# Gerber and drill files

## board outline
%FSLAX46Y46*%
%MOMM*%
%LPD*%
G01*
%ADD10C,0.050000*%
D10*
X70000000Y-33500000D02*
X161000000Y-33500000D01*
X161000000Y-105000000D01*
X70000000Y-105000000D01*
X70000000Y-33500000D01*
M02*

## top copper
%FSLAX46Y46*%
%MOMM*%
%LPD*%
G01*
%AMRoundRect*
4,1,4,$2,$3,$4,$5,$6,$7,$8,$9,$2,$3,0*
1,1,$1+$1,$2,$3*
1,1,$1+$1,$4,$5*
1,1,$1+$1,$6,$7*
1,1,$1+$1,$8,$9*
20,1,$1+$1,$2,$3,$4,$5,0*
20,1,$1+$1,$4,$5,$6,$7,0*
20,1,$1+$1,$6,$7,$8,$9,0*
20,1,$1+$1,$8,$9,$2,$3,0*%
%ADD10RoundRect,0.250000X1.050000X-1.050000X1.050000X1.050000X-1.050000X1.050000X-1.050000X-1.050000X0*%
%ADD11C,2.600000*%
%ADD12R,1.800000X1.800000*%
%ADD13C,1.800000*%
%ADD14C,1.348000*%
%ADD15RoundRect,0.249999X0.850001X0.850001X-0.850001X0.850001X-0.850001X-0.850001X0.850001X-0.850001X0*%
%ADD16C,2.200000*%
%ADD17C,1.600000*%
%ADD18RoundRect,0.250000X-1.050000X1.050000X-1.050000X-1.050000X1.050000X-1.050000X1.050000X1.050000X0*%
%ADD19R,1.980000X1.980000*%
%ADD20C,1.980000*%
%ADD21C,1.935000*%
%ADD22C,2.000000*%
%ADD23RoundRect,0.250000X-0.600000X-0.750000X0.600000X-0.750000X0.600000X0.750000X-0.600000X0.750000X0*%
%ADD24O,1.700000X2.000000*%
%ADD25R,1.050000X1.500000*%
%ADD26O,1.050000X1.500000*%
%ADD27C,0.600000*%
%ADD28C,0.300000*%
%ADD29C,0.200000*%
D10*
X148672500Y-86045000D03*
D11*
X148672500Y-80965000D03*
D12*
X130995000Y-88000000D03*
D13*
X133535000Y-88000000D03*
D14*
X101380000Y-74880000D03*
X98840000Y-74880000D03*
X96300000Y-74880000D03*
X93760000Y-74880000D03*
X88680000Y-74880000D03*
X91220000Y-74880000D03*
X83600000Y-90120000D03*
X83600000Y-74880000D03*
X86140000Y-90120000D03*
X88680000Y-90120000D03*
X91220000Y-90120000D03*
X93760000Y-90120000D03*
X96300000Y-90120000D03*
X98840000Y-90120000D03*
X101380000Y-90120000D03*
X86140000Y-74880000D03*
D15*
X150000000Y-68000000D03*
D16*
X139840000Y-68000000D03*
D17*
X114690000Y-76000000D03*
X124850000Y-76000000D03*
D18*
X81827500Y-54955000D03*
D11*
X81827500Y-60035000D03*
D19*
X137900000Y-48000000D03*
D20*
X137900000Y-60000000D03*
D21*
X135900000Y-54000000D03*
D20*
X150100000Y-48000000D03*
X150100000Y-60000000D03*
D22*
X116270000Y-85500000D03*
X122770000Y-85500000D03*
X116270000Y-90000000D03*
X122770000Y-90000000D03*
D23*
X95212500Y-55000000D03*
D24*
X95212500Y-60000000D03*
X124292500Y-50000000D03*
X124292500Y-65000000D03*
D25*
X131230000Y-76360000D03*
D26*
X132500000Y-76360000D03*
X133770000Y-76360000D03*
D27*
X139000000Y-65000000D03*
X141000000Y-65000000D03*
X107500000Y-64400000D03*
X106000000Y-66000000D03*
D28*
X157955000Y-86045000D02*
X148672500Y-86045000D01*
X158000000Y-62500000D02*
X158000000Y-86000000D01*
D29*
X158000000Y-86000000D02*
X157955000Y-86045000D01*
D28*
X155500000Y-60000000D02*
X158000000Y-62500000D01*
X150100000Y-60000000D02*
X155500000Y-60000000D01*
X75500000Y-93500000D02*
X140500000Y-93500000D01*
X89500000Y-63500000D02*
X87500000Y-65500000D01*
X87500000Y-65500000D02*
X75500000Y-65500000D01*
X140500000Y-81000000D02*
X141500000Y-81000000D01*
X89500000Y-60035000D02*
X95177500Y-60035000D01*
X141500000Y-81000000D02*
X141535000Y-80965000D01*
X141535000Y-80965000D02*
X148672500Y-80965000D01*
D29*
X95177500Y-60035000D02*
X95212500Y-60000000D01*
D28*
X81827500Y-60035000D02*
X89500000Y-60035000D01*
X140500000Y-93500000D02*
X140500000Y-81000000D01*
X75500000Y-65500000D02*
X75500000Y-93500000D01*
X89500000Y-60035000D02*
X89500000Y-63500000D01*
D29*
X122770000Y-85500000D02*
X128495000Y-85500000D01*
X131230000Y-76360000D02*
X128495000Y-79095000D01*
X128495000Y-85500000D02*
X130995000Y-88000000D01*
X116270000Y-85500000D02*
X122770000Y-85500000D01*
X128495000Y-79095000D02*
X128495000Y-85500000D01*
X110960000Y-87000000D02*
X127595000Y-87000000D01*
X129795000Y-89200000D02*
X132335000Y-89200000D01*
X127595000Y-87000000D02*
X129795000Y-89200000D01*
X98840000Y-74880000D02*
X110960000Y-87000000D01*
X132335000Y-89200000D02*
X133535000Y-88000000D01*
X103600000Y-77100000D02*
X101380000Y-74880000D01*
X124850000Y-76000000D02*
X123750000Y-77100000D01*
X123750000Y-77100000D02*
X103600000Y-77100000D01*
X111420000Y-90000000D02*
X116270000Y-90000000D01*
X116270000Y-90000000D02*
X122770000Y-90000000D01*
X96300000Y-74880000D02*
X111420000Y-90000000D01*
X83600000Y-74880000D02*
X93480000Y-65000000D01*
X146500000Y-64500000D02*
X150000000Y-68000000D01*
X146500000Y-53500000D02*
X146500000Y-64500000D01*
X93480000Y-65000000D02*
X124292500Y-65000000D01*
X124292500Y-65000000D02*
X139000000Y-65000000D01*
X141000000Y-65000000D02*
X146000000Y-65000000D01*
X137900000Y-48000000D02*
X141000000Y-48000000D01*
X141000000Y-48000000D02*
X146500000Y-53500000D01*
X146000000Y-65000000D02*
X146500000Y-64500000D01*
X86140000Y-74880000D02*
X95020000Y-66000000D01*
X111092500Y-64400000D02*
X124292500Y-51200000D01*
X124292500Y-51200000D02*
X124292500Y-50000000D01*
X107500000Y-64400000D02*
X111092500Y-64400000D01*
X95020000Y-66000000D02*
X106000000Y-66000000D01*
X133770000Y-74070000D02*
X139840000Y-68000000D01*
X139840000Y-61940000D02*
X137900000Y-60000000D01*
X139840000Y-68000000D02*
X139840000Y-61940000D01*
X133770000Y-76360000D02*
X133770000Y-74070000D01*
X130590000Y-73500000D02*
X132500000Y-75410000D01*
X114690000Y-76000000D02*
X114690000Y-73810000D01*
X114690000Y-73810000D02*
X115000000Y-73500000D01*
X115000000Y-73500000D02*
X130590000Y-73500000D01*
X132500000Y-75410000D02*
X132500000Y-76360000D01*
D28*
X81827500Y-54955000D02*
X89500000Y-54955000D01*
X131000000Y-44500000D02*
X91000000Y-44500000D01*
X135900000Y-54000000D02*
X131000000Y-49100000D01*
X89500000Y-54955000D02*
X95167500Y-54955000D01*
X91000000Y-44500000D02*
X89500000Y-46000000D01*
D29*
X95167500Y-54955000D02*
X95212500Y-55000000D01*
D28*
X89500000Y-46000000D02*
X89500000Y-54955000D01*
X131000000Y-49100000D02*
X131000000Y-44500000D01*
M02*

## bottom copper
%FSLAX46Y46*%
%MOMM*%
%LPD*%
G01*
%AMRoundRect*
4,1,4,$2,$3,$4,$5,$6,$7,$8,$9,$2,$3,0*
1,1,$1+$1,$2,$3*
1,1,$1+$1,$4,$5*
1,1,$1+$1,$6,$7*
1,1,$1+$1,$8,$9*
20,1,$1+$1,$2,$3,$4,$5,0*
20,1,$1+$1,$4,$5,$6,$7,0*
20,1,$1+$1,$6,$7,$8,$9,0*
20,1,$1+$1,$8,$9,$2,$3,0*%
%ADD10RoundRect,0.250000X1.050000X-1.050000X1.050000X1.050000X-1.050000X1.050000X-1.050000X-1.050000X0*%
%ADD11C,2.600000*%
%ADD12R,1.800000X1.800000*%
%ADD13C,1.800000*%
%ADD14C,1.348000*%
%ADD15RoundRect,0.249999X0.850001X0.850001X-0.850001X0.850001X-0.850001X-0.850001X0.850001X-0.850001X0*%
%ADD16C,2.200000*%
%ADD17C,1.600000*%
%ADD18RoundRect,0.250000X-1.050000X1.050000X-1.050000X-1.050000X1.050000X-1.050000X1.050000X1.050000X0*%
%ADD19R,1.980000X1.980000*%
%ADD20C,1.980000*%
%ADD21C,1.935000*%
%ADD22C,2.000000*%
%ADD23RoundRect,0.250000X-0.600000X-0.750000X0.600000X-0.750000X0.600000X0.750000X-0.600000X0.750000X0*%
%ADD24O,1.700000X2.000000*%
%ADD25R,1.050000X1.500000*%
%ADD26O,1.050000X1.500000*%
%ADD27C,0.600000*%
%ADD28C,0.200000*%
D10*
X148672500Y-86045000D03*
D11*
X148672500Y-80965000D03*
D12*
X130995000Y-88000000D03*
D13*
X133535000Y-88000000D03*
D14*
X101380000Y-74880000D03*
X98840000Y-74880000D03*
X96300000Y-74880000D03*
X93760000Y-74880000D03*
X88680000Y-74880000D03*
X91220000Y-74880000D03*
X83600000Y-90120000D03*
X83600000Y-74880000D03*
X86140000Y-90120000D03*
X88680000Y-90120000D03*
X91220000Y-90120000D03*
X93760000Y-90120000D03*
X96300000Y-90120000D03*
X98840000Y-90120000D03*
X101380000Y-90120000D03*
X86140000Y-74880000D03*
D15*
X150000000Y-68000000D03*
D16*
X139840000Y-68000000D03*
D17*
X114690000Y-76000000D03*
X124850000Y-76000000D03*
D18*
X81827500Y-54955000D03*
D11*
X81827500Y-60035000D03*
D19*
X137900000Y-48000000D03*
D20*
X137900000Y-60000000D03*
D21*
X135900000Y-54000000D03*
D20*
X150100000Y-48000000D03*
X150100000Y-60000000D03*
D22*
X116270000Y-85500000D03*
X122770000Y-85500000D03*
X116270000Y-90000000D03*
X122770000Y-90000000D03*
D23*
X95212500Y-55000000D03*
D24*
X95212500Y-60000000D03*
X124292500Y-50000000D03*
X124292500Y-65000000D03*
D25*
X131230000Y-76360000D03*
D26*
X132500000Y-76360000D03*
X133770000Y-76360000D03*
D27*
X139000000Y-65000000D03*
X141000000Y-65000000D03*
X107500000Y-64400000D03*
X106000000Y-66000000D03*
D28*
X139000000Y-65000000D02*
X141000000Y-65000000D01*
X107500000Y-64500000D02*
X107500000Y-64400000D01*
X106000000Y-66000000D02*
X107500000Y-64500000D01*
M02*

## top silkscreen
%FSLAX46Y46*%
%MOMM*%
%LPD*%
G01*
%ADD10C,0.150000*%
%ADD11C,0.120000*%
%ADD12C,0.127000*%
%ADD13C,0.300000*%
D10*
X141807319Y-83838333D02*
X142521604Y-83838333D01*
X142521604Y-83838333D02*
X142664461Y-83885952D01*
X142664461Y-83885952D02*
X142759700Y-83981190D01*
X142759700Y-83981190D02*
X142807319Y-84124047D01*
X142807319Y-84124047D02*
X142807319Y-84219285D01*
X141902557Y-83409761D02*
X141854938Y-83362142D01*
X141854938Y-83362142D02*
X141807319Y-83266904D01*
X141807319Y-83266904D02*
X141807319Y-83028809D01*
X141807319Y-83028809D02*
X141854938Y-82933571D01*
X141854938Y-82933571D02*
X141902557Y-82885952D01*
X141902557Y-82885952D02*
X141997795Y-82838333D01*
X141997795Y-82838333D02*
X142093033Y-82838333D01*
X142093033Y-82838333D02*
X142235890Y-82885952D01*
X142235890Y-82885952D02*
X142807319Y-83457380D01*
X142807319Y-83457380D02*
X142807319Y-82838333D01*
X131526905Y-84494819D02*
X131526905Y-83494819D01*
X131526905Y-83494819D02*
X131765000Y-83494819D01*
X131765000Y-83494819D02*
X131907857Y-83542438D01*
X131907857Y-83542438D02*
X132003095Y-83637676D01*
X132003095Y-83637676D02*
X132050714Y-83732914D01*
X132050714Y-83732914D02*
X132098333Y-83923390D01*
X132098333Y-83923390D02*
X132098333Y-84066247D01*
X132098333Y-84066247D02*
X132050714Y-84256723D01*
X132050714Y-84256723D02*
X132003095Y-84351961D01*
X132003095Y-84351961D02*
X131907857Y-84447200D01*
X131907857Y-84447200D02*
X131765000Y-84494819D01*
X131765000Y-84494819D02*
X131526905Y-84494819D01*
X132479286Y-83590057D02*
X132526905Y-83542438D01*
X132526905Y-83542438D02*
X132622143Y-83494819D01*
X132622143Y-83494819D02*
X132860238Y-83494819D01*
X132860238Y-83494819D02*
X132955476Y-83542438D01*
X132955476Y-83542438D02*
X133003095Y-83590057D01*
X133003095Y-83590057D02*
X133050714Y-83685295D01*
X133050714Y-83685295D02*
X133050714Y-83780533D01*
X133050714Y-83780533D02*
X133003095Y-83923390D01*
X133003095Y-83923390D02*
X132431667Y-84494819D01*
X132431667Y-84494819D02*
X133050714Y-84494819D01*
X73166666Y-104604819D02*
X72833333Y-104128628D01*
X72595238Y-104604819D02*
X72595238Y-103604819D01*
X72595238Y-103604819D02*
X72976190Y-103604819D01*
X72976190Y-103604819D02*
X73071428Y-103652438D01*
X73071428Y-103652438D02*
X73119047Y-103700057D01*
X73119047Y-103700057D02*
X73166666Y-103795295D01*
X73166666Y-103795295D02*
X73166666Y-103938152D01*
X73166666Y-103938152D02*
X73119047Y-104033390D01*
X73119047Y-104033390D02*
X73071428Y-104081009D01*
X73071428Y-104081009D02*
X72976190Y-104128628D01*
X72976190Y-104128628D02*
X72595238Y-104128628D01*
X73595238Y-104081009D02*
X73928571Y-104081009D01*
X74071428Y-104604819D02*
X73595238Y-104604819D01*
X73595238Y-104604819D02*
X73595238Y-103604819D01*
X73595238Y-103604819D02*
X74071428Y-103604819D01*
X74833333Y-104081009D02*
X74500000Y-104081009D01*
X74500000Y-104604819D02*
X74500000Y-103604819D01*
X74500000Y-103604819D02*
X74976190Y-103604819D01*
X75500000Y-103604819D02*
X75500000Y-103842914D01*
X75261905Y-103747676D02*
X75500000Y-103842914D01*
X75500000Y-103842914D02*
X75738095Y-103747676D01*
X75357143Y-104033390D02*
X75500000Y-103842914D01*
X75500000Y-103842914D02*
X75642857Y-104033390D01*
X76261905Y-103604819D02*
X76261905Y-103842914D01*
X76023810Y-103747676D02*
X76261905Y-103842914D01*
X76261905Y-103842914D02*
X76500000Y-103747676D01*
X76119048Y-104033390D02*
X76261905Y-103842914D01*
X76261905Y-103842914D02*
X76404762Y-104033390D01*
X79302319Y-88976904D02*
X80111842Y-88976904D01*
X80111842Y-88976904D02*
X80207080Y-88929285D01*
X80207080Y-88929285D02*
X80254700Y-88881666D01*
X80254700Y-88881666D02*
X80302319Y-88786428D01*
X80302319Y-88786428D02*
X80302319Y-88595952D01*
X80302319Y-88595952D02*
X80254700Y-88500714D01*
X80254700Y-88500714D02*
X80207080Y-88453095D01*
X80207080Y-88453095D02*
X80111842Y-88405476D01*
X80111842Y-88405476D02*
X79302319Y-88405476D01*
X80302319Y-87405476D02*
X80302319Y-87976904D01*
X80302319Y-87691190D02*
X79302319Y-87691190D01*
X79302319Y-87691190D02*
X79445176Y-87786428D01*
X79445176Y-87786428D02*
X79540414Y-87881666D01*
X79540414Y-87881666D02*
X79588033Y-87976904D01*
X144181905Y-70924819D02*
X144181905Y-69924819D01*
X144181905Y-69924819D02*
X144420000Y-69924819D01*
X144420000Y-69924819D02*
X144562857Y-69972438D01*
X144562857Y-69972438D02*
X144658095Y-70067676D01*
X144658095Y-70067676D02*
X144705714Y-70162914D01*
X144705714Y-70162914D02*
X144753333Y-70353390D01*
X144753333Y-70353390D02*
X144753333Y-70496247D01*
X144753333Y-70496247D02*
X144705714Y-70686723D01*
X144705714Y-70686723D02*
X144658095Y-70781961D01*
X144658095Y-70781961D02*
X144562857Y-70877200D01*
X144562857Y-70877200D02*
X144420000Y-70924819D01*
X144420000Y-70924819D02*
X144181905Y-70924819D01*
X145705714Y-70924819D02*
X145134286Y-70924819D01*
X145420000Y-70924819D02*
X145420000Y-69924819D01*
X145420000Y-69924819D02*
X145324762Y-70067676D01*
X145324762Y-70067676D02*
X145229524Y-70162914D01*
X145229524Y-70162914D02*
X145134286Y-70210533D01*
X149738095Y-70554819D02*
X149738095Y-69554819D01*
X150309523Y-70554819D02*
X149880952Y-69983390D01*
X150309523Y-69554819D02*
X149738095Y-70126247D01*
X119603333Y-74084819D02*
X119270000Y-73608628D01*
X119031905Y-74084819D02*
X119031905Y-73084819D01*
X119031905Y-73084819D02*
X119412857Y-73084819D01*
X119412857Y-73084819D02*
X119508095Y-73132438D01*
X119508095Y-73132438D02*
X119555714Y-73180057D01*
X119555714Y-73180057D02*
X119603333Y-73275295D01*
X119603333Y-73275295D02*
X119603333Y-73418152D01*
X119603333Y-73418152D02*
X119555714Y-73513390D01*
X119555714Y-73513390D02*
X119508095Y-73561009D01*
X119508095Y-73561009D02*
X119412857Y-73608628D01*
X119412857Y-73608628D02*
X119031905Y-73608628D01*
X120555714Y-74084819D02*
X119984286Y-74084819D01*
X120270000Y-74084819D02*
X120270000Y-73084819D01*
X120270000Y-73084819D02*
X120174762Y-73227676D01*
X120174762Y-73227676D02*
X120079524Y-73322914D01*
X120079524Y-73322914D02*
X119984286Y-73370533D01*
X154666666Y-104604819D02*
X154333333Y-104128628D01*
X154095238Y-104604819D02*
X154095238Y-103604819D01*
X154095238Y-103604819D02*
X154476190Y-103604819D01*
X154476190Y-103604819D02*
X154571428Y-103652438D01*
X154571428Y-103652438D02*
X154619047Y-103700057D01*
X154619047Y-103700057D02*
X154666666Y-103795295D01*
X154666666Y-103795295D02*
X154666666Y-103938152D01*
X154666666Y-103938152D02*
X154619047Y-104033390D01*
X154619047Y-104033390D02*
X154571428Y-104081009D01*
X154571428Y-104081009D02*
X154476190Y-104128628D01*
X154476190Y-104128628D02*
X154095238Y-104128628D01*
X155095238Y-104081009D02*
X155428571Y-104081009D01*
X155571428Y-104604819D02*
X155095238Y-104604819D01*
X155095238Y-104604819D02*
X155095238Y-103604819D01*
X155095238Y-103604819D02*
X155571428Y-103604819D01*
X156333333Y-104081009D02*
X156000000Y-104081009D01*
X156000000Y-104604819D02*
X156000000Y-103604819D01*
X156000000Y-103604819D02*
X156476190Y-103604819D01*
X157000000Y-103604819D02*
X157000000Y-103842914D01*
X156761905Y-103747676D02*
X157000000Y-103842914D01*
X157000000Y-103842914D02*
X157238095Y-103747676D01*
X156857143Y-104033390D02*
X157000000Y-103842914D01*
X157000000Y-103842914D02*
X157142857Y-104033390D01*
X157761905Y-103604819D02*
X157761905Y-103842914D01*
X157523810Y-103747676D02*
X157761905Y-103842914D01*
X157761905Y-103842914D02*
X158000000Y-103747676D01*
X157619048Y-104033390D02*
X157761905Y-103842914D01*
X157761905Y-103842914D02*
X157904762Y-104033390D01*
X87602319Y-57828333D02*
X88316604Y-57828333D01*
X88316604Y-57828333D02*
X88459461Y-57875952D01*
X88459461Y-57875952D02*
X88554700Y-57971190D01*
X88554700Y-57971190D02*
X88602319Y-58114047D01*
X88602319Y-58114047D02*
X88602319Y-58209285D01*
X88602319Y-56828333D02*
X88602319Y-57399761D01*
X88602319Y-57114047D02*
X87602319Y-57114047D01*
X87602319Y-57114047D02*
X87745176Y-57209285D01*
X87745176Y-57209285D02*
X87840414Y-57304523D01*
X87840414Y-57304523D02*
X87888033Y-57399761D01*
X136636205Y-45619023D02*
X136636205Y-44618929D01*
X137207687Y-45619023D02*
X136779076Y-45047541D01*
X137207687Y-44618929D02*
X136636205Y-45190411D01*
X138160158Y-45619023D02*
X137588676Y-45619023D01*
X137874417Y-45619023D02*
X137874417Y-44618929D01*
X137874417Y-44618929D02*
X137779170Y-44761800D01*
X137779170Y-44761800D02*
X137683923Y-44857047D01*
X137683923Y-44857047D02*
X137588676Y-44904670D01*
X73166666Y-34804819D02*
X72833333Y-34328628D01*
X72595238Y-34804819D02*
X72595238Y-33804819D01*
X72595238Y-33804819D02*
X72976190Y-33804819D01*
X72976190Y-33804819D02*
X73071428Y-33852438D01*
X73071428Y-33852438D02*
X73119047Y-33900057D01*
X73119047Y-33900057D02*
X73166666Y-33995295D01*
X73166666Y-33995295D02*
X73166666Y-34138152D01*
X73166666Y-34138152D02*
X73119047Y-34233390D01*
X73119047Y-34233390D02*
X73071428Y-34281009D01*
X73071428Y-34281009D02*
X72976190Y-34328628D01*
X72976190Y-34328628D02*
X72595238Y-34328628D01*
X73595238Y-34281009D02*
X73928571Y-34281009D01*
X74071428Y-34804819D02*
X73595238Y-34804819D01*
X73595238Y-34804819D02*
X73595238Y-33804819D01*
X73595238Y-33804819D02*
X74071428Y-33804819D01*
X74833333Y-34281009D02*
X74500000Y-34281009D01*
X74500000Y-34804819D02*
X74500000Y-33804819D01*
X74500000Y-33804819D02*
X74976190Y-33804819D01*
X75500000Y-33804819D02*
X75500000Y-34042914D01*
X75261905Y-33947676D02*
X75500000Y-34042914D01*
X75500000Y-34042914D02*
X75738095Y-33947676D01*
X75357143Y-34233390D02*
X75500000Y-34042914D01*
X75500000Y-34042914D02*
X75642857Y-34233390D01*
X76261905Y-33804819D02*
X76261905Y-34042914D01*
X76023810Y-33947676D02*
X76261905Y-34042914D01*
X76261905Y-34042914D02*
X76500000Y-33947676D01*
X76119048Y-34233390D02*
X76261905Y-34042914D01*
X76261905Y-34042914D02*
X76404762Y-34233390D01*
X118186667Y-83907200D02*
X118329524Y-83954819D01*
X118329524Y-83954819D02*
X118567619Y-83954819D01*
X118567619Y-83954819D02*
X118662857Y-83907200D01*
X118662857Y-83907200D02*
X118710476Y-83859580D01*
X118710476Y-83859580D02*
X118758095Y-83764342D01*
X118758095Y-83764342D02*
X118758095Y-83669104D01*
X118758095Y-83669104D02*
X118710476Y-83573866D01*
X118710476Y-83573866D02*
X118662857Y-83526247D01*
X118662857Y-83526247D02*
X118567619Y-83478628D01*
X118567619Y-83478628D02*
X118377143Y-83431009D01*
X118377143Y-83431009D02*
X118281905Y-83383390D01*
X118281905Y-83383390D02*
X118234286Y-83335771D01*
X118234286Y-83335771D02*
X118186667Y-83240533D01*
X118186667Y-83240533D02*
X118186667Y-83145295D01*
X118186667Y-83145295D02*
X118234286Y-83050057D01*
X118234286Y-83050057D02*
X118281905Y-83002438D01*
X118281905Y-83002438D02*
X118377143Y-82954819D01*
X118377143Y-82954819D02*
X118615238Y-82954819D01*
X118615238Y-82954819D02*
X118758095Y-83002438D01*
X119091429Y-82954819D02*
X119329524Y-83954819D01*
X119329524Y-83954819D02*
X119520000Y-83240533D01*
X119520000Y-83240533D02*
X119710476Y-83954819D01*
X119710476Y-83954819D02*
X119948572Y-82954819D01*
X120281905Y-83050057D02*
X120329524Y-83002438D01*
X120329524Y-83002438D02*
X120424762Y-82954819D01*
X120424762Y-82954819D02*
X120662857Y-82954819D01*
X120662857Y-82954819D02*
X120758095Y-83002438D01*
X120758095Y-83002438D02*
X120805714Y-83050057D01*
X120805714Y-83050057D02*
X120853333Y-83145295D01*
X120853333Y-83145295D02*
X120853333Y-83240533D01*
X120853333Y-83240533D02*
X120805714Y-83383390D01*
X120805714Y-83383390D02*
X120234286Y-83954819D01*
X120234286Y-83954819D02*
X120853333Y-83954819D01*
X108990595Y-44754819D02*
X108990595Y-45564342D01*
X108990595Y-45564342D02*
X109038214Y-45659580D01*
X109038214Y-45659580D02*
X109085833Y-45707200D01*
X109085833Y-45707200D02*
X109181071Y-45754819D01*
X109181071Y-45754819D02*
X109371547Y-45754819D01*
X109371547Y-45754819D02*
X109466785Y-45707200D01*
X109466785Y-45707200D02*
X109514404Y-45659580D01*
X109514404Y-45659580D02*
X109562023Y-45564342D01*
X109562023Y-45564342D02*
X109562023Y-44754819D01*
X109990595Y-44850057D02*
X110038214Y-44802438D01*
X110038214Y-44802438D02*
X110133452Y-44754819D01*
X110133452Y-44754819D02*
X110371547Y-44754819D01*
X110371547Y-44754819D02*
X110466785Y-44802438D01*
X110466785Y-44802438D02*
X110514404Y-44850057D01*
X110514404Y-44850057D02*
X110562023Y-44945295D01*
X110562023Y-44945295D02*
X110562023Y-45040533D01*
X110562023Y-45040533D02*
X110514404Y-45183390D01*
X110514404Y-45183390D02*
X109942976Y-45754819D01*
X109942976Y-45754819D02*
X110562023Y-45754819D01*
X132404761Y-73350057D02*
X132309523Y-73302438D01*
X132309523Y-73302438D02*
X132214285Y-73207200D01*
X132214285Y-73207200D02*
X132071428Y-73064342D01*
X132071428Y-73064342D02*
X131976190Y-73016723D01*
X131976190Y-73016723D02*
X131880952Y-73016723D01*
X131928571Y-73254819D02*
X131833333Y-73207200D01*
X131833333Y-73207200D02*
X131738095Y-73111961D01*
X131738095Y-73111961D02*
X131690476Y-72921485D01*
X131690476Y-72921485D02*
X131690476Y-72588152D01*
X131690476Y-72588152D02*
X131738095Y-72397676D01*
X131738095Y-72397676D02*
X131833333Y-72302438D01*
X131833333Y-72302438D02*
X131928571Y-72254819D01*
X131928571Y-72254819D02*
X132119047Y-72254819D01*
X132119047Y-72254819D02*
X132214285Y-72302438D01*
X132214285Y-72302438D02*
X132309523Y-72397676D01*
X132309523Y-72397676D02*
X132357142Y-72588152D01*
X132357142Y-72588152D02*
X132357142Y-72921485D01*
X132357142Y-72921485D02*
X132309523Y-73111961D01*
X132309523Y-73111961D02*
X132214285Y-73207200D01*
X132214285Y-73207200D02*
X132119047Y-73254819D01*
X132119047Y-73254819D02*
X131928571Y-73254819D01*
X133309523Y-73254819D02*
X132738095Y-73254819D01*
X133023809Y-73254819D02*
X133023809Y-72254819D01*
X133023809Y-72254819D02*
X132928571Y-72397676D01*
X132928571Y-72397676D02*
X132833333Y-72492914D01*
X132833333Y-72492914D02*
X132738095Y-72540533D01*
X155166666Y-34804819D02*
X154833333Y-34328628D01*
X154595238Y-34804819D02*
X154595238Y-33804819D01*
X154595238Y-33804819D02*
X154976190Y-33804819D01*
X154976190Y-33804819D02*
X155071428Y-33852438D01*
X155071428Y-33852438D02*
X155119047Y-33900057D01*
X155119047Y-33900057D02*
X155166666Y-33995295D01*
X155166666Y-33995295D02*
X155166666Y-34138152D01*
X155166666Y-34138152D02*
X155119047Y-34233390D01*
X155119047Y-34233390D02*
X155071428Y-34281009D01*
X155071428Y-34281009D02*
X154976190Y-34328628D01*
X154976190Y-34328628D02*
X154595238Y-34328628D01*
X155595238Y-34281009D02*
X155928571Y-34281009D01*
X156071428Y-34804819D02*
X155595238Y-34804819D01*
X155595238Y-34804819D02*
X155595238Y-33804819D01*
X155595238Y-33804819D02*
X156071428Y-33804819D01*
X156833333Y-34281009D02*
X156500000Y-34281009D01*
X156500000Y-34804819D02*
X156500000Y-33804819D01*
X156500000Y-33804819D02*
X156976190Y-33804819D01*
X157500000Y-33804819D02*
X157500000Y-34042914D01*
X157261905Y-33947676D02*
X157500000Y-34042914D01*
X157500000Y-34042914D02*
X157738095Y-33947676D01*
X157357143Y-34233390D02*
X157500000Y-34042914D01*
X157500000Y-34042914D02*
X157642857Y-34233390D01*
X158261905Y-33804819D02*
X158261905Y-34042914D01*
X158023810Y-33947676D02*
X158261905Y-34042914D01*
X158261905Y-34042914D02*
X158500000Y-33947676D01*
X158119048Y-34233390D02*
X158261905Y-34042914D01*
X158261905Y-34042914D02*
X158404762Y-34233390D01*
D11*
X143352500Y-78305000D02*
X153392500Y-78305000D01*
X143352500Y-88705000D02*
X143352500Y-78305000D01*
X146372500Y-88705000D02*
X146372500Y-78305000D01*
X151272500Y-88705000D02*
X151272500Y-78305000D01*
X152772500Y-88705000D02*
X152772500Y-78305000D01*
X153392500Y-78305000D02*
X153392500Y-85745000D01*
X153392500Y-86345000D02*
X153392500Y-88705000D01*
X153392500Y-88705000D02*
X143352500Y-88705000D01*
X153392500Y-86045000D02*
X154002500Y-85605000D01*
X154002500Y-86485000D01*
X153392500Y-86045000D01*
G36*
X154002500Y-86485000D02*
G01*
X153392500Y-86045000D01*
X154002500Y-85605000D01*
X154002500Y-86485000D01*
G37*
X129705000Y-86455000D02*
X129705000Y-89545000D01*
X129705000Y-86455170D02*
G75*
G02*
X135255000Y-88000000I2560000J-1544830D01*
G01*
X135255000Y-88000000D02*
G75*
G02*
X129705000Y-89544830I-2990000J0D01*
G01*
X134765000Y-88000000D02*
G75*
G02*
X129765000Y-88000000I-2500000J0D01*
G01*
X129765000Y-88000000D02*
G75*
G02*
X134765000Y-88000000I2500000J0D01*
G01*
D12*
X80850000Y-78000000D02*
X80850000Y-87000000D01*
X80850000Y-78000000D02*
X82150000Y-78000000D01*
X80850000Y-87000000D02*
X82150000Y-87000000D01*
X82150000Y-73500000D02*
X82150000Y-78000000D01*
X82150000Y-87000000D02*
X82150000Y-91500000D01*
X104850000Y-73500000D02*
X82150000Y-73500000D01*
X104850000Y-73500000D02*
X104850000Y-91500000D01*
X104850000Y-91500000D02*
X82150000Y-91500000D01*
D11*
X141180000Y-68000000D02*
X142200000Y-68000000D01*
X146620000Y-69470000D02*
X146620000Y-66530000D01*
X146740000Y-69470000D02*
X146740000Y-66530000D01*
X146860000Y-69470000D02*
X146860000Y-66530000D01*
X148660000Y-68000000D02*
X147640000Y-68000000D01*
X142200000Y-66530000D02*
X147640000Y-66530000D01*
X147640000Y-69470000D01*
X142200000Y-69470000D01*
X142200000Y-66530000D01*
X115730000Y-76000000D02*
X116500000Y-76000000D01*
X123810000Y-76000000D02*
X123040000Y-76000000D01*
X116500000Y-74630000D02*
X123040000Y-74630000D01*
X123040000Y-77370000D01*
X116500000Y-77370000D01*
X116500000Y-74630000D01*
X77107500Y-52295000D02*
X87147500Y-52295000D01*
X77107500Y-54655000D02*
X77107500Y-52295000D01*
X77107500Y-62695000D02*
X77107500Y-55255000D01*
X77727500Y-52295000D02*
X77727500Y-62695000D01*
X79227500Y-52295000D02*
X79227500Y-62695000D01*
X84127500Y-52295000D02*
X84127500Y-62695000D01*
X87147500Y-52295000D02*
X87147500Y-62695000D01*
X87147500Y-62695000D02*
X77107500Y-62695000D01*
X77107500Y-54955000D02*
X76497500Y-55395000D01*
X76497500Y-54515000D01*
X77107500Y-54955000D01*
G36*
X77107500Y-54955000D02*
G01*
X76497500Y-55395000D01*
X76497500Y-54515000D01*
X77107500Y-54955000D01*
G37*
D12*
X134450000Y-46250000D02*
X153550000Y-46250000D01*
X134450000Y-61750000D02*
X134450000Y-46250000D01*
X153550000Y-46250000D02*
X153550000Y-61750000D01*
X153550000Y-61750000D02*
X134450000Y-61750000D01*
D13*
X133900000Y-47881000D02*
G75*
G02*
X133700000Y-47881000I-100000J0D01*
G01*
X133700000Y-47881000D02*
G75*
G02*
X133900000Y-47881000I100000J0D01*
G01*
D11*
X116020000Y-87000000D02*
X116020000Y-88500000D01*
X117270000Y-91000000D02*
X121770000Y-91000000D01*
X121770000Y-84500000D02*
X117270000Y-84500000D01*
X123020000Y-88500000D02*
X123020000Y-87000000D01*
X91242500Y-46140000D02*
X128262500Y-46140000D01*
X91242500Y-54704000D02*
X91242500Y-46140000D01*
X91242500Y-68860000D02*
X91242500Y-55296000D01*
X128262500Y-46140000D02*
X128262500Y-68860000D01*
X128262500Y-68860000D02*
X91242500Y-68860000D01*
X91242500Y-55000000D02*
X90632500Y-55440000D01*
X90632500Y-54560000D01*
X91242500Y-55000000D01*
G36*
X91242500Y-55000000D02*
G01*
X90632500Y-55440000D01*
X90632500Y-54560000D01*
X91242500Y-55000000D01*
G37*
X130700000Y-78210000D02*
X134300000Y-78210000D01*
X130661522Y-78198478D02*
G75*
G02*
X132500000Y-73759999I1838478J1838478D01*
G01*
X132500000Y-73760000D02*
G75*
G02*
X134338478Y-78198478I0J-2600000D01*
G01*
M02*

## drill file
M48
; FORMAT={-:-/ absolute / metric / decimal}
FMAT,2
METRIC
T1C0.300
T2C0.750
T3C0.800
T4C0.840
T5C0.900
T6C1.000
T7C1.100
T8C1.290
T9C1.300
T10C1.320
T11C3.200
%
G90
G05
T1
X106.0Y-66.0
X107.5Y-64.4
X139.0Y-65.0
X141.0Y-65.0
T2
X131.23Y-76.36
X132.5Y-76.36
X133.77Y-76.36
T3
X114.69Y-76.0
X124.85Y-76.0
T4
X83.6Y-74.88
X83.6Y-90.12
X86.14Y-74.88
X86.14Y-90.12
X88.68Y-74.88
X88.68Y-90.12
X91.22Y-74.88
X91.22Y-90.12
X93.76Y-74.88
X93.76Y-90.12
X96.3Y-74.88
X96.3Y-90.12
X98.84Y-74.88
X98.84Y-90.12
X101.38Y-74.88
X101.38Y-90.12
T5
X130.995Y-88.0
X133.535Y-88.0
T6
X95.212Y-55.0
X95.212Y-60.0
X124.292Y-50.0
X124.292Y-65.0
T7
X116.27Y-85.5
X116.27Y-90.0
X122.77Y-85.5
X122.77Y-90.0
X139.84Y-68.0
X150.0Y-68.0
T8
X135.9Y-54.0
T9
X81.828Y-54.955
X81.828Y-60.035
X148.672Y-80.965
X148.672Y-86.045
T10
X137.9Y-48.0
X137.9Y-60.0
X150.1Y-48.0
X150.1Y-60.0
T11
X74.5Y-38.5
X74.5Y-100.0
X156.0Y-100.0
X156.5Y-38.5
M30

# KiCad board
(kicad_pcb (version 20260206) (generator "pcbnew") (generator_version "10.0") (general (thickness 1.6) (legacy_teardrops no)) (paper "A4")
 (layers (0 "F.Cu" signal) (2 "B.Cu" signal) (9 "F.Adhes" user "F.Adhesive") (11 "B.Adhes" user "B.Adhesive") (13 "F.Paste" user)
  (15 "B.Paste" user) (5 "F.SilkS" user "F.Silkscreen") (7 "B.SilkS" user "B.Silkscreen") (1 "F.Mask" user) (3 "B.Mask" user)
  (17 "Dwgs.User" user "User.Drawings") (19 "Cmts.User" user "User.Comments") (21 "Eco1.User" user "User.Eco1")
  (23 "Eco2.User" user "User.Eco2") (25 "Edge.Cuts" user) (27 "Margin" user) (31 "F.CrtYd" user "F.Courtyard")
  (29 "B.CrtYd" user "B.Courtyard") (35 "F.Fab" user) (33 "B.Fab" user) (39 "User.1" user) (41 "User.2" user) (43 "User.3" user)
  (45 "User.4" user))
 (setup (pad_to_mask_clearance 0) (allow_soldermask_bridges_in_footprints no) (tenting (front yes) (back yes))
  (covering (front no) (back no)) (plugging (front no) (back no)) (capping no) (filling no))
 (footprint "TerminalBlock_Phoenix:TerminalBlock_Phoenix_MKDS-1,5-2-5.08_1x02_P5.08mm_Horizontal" (layer "F.Cu") (at 148.6725 86.045 90)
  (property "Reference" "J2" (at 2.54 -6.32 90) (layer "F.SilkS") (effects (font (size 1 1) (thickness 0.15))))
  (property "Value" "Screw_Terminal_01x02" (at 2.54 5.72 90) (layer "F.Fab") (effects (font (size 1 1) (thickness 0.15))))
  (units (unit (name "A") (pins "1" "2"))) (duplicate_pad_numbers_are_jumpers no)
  (fp_line (start 7.74 -5.32) (end 7.74 4.72) (stroke (width 0.12) (type solid)) (layer "F.SilkS"))
  (fp_line (start -2.66 -5.32) (end 7.74 -5.32) (stroke (width 0.12) (type solid)) (layer "F.SilkS"))
  (fp_line (start -2.66 -2.3) (end 7.74 -2.3) (stroke (width 0.12) (type solid)) (layer "F.SilkS"))
  (fp_line (start -2.66 2.6) (end 7.74 2.6) (stroke (width 0.12) (type solid)) (layer "F.SilkS"))
  (fp_line (start -2.66 4.1) (end 7.74 4.1) (stroke (width 0.12) (type solid)) (layer "F.SilkS"))
  (fp_line (start 7.74 4.72) (end 0.3 4.72) (stroke (width 0.12) (type solid)) (layer "F.SilkS"))
  (fp_line (start -0.3 4.72) (end -2.66 4.72) (stroke (width 0.12) (type solid)) (layer "F.SilkS"))
  (fp_line (start -2.66 4.72) (end -2.66 -5.32) (stroke (width 0.12) (type solid)) (layer "F.SilkS"))
  (fp_poly (pts (xy 0 4.72) (xy 0.44 5.33) (xy -0.44 5.33)) (stroke (width 0.12) (type solid)) (fill yes) (layer "F.SilkS"))
  (pad "1" thru_hole roundrect (at 0 0 90) (size 2.6 2.6) (drill 1.3) (layers "*.Cu" "*.Mask") (remove_unused_layers no)
   (roundrect_rratio 0.096154) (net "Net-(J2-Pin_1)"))
  (pad "2" thru_hole circle (at 5.08 0 90) (size 2.6 2.6) (drill 1.3) (layers "*.Cu" "*.Mask") (remove_unused_layers no)
   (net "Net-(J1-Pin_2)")))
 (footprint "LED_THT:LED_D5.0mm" (layer "F.Cu") (at 130.995 88)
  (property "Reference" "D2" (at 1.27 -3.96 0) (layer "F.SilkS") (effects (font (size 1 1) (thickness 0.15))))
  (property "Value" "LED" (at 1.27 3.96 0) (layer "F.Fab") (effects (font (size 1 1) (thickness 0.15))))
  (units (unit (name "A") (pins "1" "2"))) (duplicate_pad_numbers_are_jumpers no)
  (fp_line (start -1.29 -1.545) (end -1.29 1.545) (stroke (width 0.12) (type solid)) (layer "F.SilkS"))
  (fp_arc (start -1.29 -1.54483) (mid 2.071779 -2.880495) (end 4.26 0) (stroke (width 0.12) (type solid)) (layer "F.SilkS"))
  (fp_arc (start 4.26 0) (mid 2.071779 2.880495) (end -1.29 1.54483) (stroke (width 0.12) (type solid)) (layer "F.SilkS"))
  (fp_circle (center 1.27 0) (end 3.77 0) (stroke (width 0.12) (type solid)) (fill no) (layer "F.SilkS"))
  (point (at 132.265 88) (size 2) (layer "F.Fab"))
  (pad "1" thru_hole rect (at 0 0) (size 1.8 1.8) (drill 0.9) (layers "*.Cu" "*.Mask") (remove_unused_layers no) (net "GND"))
  (pad "2" thru_hole circle (at 2.54 0) (size 1.8 1.8) (drill 0.9) (layers "*.Cu" "*.Mask") (remove_unused_layers no) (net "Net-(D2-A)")))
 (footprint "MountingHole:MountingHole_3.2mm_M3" (layer "F.Cu") (at 74.5 100 180)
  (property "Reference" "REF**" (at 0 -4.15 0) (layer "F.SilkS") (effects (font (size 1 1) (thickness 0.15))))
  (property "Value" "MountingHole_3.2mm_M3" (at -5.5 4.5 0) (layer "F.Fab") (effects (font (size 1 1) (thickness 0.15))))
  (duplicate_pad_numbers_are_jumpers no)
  (pad "" np_thru_hole circle (at 0 0 180) (size 3.2 3.2) (drill 3.2) (layers "*.Cu" "*.Mask")))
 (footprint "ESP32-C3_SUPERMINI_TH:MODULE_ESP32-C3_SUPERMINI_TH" (layer "F.Cu") (at 93.5 82.5 90)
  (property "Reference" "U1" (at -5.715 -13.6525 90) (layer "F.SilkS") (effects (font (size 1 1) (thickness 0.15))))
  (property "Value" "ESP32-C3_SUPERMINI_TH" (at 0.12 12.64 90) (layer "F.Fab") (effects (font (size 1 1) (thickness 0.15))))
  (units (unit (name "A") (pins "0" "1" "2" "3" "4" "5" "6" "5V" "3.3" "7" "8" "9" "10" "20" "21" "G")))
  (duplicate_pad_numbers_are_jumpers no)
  (fp_line (start 4.5 -12.65) (end -4.5 -12.65) (stroke (width 0.127) (type solid)) (layer "F.SilkS"))
  (fp_line (start 4.5 -12.65) (end 4.5 -11.35) (stroke (width 0.127) (type solid)) (layer "F.SilkS"))
  (fp_line (start -4.5 -12.65) (end -4.5 -11.35) (stroke (width 0.127) (type solid)) (layer "F.SilkS"))
  (fp_line (start 9 -11.35) (end 4.5 -11.35) (stroke (width 0.127) (type solid)) (layer "F.SilkS"))
  (fp_line (start -4.5 -11.35) (end -9 -11.35) (stroke (width 0.127) (type solid)) (layer "F.SilkS"))
  (fp_line (start 9 11.35) (end 9 -11.35) (stroke (width 0.127) (type solid)) (layer "F.SilkS"))
  (fp_line (start 9 11.35) (end -9 11.35) (stroke (width 0.127) (type solid)) (layer "F.SilkS"))
  (fp_line (start -9 11.35) (end -9 -11.35) (stroke (width 0.127) (type solid)) (layer "F.SilkS"))
  (pad "0" thru_hole circle (at 7.62 7.88 90) (size 1.348 1.348) (drill 0.84) (layers "*.Cu" "*.Mask") (remove_unused_layers no)
   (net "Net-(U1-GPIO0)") (solder_mask_margin 0.102))
  (pad "1" thru_hole circle (at 7.62 5.34 90) (size 1.348 1.348) (drill 0.84) (layers "*.Cu" "*.Mask") (remove_unused_layers no)
   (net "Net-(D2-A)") (solder_mask_margin 0.102))
  (pad "2" thru_hole circle (at 7.62 2.8 90) (size 1.348 1.348) (drill 0.84) (layers "*.Cu" "*.Mask") (remove_unused_layers no)
   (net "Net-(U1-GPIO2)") (solder_mask_margin 0.102))
  (pad "3" thru_hole circle (at 7.62 0.26 90) (size 1.348 1.348) (drill 0.84) (layers "*.Cu" "*.Mask") (remove_unused_layers no)
   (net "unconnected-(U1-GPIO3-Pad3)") (solder_mask_margin 0.102))
  (pad "3.3" thru_hole circle (at 7.62 -4.82 90) (size 1.348 1.348) (drill 0.84) (layers "*.Cu" "*.Mask") (remove_unused_layers no)
   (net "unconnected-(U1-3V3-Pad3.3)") (solder_mask_margin 0.102))
  (pad "4" thru_hole circle (at 7.62 -2.28 90) (size 1.348 1.348) (drill 0.84) (layers "*.Cu" "*.Mask") (remove_unused_layers no)
   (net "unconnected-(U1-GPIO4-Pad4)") (solder_mask_margin 0.102))
  (pad "5" thru_hole circle (at -7.62 -9.9 90) (size 1.348 1.348) (drill 0.84) (layers "*.Cu" "*.Mask") (remove_unused_layers no)
   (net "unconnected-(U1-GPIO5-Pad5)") (solder_mask_margin 0.102))
  (pad "5V" thru_hole circle (at 7.62 -9.9 90) (size 1.348 1.348) (drill 0.84) (layers "*.Cu" "*.Mask") (remove_unused_layers no)
   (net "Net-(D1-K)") (solder_mask_margin 0.102))
  (pad "6" thru_hole circle (at -7.62 -7.36 90) (size 1.348 1.348) (drill 0.84) (layers "*.Cu" "*.Mask") (remove_unused_layers no)
   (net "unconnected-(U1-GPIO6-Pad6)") (solder_mask_margin 0.102))
  (pad "7" thru_hole circle (at -7.62 -4.82 90) (size 1.348 1.348) (drill 0.84) (layers "*.Cu" "*.Mask") (remove_unused_layers no)
   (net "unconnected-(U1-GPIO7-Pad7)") (solder_mask_margin 0.102))
  (pad "8" thru_hole circle (at -7.62 -2.28 90) (size 1.348 1.348) (drill 0.84) (layers "*.Cu" "*.Mask") (remove_unused_layers no)
   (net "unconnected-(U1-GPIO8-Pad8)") (solder_mask_margin 0.102))
  (pad "9" thru_hole circle (at -7.62 0.26 90) (size 1.348 1.348) (drill 0.84) (layers "*.Cu" "*.Mask") (remove_unused_layers no)
   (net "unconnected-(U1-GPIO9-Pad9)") (solder_mask_margin 0.102))
  (pad "10" thru_hole circle (at -7.62 2.8 90) (size 1.348 1.348) (drill 0.84) (layers "*.Cu" "*.Mask") (remove_unused_layers no)
   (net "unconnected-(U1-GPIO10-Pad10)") (solder_mask_margin 0.102))
  (pad "20" thru_hole circle (at -7.62 5.34 90) (size 1.348 1.348) (drill 0.84) (layers "*.Cu" "*.Mask") (remove_unused_layers no)
   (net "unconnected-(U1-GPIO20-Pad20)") (solder_mask_margin 0.102))
  (pad "21" thru_hole circle (at -7.62 7.88 90) (size 1.348 1.348) (drill 0.84) (layers "*.Cu" "*.Mask") (remove_unused_layers no)
   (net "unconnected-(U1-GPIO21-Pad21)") (solder_mask_margin 0.102))
  (pad "G" thru_hole circle (at 7.62 -7.36 90) (size 1.348 1.348) (drill 0.84) (layers "*.Cu" "*.Mask") (remove_unused_layers no)
   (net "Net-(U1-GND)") (solder_mask_margin 0.102)))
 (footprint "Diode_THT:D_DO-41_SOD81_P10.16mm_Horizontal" (layer "F.Cu") (at 150 68 180)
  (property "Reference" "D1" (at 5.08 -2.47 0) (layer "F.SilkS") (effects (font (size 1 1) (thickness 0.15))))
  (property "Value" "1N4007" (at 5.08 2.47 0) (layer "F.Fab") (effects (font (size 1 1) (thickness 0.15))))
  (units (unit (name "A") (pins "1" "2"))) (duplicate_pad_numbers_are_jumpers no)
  (fp_line (start 8.82 0) (end 7.8 0) (stroke (width 0.12) (type solid)) (layer "F.SilkS"))
  (fp_line (start 3.38 -1.47) (end 3.38 1.47) (stroke (width 0.12) (type solid)) (layer "F.SilkS"))
  (fp_line (start 3.26 -1.47) (end 3.26 1.47) (stroke (width 0.12) (type solid)) (layer "F.SilkS"))
  (fp_line (start 3.14 -1.47) (end 3.14 1.47) (stroke (width 0.12) (type solid)) (layer "F.SilkS"))
  (fp_line (start 1.34 0) (end 2.36 0) (stroke (width 0.12) (type solid)) (layer "F.SilkS"))
  (fp_rect (start 2.36 -1.47) (end 7.8 1.47) (stroke (width 0.12) (type solid)) (fill no) (layer "F.SilkS"))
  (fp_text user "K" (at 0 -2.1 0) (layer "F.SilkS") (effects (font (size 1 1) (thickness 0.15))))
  (pad "1" thru_hole roundrect (at 0 0 180) (size 2.2 2.2) (drill 1.1) (layers "*.Cu" "*.Mask") (remove_unused_layers no)
   (roundrect_rratio 0.113636) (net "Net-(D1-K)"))
  (pad "2" thru_hole circle (at 10.16 0 180) (size 2.2 2.2) (drill 1.1) (layers "*.Cu" "*.Mask") (remove_unused_layers no)
   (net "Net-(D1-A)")))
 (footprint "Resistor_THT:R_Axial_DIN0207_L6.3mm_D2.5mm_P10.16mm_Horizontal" (layer "F.Cu") (at 114.69 76)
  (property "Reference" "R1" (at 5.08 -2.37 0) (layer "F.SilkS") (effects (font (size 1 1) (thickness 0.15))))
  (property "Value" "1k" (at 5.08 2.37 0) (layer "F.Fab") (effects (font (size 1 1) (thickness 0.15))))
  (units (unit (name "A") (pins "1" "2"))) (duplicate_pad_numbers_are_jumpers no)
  (fp_line (start 1.04 0) (end 1.81 0) (stroke (width 0.12) (type solid)) (layer "F.SilkS"))
  (fp_line (start 9.12 0) (end 8.35 0) (stroke (width 0.12) (type solid)) (layer "F.SilkS"))
  (fp_rect (start 1.81 -1.37) (end 8.35 1.37) (stroke (width 0.12) (type solid)) (fill no) (layer "F.SilkS"))
  (pad "1" thru_hole circle (at 0 0) (size 1.6 1.6) (drill 0.8) (layers "*.Cu" "*.Mask") (remove_unused_layers no) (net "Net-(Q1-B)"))
  (pad "2" thru_hole circle (at 10.16 0) (size 1.6 1.6) (drill 0.8) (layers "*.Cu" "*.Mask") (remove_unused_layers no)
   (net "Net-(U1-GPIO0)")))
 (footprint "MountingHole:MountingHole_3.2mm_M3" (layer "F.Cu") (at 156 100 180)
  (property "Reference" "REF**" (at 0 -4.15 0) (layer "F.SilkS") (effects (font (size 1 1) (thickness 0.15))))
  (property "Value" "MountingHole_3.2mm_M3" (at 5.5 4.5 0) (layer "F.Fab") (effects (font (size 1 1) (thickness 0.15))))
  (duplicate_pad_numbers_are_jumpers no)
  (pad "" np_thru_hole circle (at 0 0 180) (size 3.2 3.2) (drill 3.2) (layers "*.Cu" "*.Mask")))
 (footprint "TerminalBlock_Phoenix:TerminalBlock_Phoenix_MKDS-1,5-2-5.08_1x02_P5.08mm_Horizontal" (layer "F.Cu") (at 81.8275 54.955 -90)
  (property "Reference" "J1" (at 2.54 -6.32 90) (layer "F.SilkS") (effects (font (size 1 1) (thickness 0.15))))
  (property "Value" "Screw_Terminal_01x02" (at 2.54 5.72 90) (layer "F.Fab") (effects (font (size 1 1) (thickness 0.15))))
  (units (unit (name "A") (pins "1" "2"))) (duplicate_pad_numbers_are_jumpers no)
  (fp_line (start -2.66 4.72) (end -2.66 -5.32) (stroke (width 0.12) (type solid)) (layer "F.SilkS"))
  (fp_line (start -0.3 4.72) (end -2.66 4.72) (stroke (width 0.12) (type solid)) (layer "F.SilkS"))
  (fp_line (start 7.74 4.72) (end 0.3 4.72) (stroke (width 0.12) (type solid)) (layer "F.SilkS"))
  (fp_line (start -2.66 4.1) (end 7.74 4.1) (stroke (width 0.12) (type solid)) (layer "F.SilkS"))
  (fp_line (start -2.66 2.6) (end 7.74 2.6) (stroke (width 0.12) (type solid)) (layer "F.SilkS"))
  (fp_line (start -2.66 -2.3) (end 7.74 -2.3) (stroke (width 0.12) (type solid)) (layer "F.SilkS"))
  (fp_line (start -2.66 -5.32) (end 7.74 -5.32) (stroke (width 0.12) (type solid)) (layer "F.SilkS"))
  (fp_line (start 7.74 -5.32) (end 7.74 4.72) (stroke (width 0.12) (type solid)) (layer "F.SilkS"))
  (fp_poly (pts (xy 0 4.72) (xy 0.44 5.33) (xy -0.44 5.33)) (stroke (width 0.12) (type solid)) (fill yes) (layer "F.SilkS"))
  (pad "1" thru_hole roundrect (at 0 0 270) (size 2.6 2.6) (drill 1.3) (layers "*.Cu" "*.Mask") (remove_unused_layers no)
   (roundrect_rratio 0.096154) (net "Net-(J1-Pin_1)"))
  (pad "2" thru_hole circle (at 5.08 0 270) (size 2.6 2.6) (drill 1.3) (layers "*.Cu" "*.Mask") (remove_unused_layers no)
   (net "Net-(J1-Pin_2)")))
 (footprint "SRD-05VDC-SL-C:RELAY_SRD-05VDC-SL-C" (layer "F.Cu") (at 144 54)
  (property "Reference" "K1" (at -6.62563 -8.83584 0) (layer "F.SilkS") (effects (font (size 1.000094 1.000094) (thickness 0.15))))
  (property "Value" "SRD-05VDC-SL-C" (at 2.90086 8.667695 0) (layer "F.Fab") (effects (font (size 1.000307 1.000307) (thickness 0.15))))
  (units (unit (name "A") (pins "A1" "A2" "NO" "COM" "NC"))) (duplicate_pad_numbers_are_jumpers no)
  (fp_line (start -9.55 -7.75) (end 9.55 -7.75) (stroke (width 0.127) (type solid)) (layer "F.SilkS"))
  (fp_line (start -9.55 7.75) (end -9.55 -7.75) (stroke (width 0.127) (type solid)) (layer "F.SilkS"))
  (fp_line (start 9.55 -7.75) (end 9.55 7.75) (stroke (width 0.127) (type solid)) (layer "F.SilkS"))
  (fp_line (start 9.55 7.75) (end -9.55 7.75) (stroke (width 0.127) (type solid)) (layer "F.SilkS"))
  (fp_circle (center -10.2 -6.119) (end -10.1 -6.119) (stroke (width 0.3) (type solid)) (fill no) (layer "F.SilkS"))
  (pad "A1" thru_hole rect (at -6.1 -6) (size 1.98 1.98) (drill 1.32) (layers "*.Cu" "*.Mask") (remove_unused_layers no) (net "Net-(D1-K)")
   (solder_mask_margin 0.102))
  (pad "A2" thru_hole circle (at -6.1 6) (size 1.98 1.98) (drill 1.32) (layers "*.Cu" "*.Mask") (remove_unused_layers no) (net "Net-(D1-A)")
   (solder_mask_margin 0.102))
  (pad "COM" thru_hole circle (at -8.1 0) (size 1.935 1.935) (drill 1.29) (layers "*.Cu" "*.Mask") (remove_unused_layers no)
   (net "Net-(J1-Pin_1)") (solder_mask_margin 0.102))
  (pad "NC" thru_hole circle (at 6.1 -6) (size 1.98 1.98) (drill 1.32) (layers "*.Cu" "*.Mask") (remove_unused_layers no)
   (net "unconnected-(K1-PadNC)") (solder_mask_margin 0.102))
  (pad "NO" thru_hole circle (at 6.1 6) (size 1.98 1.98) (drill 1.32) (layers "*.Cu" "*.Mask") (remove_unused_layers no)
   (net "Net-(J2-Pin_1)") (solder_mask_margin 0.102)))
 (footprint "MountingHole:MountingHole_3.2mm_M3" (layer "F.Cu") (at 74.5 38.5)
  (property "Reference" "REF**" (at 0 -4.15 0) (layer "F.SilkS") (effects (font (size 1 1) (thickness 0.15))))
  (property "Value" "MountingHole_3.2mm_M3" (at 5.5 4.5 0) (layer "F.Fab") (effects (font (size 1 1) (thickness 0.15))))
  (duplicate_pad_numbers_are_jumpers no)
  (pad "" np_thru_hole circle (at 0 0) (size 3.2 3.2) (drill 3.2) (layers "*.Cu" "*.Mask")))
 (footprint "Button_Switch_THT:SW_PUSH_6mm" (layer "F.Cu") (at 116.27 85.5)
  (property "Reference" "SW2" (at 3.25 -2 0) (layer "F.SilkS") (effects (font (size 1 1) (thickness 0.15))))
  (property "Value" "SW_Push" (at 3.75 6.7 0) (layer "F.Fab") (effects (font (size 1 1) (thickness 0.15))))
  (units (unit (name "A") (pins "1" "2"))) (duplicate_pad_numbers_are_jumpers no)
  (fp_line (start -0.25 1.5) (end -0.25 3) (stroke (width 0.12) (type solid)) (layer "F.SilkS"))
  (fp_line (start 1 5.5) (end 5.5 5.5) (stroke (width 0.12) (type solid)) (layer "F.SilkS"))
  (fp_line (start 5.5 -1) (end 1 -1) (stroke (width 0.12) (type solid)) (layer "F.SilkS"))
  (fp_line (start 6.75 3) (end 6.75 1.5) (stroke (width 0.12) (type solid)) (layer "F.SilkS"))
  (pad "1" thru_hole circle (at 0 0 90) (size 2 2) (drill 1.1) (layers "*.Cu" "*.Mask") (remove_unused_layers no) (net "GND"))
  (pad "1" thru_hole circle (at 6.5 0 90) (size 2 2) (drill 1.1) (layers "*.Cu" "*.Mask") (remove_unused_layers no) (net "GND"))
  (pad "2" thru_hole circle (at 0 4.5 90) (size 2 2) (drill 1.1) (layers "*.Cu" "*.Mask") (remove_unused_layers no) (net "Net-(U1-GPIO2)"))
  (pad "2" thru_hole circle (at 6.5 4.5 90) (size 2 2) (drill 1.1) (layers "*.Cu" "*.Mask") (remove_unused_layers no) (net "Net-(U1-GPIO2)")))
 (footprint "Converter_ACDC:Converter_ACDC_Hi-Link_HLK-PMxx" (layer "F.Cu") (at 95.2125 55)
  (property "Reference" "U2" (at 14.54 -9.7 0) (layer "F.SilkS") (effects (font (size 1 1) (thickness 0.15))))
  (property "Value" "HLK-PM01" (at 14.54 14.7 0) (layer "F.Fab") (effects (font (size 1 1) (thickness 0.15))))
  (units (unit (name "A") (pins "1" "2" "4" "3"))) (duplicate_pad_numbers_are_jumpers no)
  (fp_line (start -3.97 -8.86) (end 33.05 -8.86) (stroke (width 0.12) (type solid)) (layer "F.SilkS"))
  (fp_line (start -3.97 -0.296) (end -3.97 -8.86) (stroke (width 0.12) (type solid)) (layer "F.SilkS"))
  (fp_line (start -3.97 13.86) (end -3.97 0.296) (stroke (width 0.12) (type solid)) (layer "F.SilkS"))
  (fp_line (start 33.05 -8.86) (end 33.05 13.86) (stroke (width 0.12) (type solid)) (layer "F.SilkS"))
  (fp_line (start 33.05 13.86) (end -3.97 13.86) (stroke (width 0.12) (type solid)) (layer "F.SilkS"))
  (fp_poly (pts (xy -3.97 0) (xy -4.58 0.44) (xy -4.58 -0.44)) (stroke (width 0.12) (type solid)) (fill yes) (layer "F.SilkS"))
  (pad "1" thru_hole roundrect (at 0 0) (size 1.7 2) (drill 1) (layers "*.Cu" "*.Mask") (remove_unused_layers no)
   (roundrect_rratio 0.147059) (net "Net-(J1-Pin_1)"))
  (pad "2" thru_hole oval (at 0 5) (size 1.7 2) (drill 1) (layers "*.Cu" "*.Mask") (remove_unused_layers no) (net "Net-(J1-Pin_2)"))
  (pad "3" thru_hole oval (at 29.08 -5) (size 1.7 2) (drill 1) (layers "*.Cu" "*.Mask") (remove_unused_layers no) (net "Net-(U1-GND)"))
  (pad "4" thru_hole oval (at 29.08 10) (size 1.7 2) (drill 1) (layers "*.Cu" "*.Mask") (remove_unused_layers no) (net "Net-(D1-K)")))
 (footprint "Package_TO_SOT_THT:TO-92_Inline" (layer "F.Cu") (at 131.23 76.36)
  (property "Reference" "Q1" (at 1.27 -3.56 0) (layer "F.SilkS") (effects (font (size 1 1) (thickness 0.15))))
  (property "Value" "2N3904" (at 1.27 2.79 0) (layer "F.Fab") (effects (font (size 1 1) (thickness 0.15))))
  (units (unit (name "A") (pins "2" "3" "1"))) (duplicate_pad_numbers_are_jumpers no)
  (fp_line (start -0.53 1.85) (end 3.07 1.85) (stroke (width 0.12) (type solid)) (layer "F.SilkS"))
  (fp_arc (start -0.568478 1.838478) (mid -1.132087 -0.994977) (end 1.27 -2.6) (stroke (width 0.12) (type solid)) (layer "F.SilkS"))
  (fp_arc (start 1.27 -2.6) (mid 3.672087 -0.994977) (end 3.108478 1.838478) (stroke (width 0.12) (type solid)) (layer "F.SilkS"))
  (pad "1" thru_hole rect (at 0 0) (size 1.05 1.5) (drill 0.75) (layers "*.Cu" "*.Mask") (remove_unused_layers no) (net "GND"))
  (pad "2" thru_hole oval (at 1.27 0) (size 1.05 1.5) (drill 0.75) (layers "*.Cu" "*.Mask") (remove_unused_layers no) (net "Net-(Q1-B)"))
  (pad "3" thru_hole oval (at 2.54 0) (size 1.05 1.5) (drill 0.75) (layers "*.Cu" "*.Mask") (remove_unused_layers no) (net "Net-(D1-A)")))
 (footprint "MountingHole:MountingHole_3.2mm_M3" (layer "F.Cu") (at 156.5 38.5)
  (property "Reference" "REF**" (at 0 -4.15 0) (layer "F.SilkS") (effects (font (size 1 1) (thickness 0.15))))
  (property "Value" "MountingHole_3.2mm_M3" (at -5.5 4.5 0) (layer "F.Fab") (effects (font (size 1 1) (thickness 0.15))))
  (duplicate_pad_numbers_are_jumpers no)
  (pad "" np_thru_hole circle (at 0 0) (size 3.2 3.2) (drill 3.2) (layers "*.Cu" "*.Mask")))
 (gr_rect (start 70 33.5) (end 161 105) (stroke (width 0.05) (type default)) (fill no) (layer "Edge.Cuts"))
 (segment (start 157.955 86.045) (end 148.6725 86.045) (width 0.3) (layer "F.Cu") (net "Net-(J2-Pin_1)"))
 (segment (start 158 62.5) (end 158 86) (width 0.3) (layer "F.Cu") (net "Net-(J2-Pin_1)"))
 (segment (start 158 86) (end 157.955 86.045) (width 0.2) (layer "F.Cu") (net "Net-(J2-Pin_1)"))
 (segment (start 155.5 60) (end 158 62.5) (width 0.3) (layer "F.Cu") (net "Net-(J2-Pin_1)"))
 (segment (start 150.1 60) (end 155.5 60) (width 0.3) (layer "F.Cu") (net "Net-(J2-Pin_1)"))
 (segment (start 75.5 93.5) (end 140.5 93.5) (width 0.3) (layer "F.Cu") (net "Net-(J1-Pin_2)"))
 (segment (start 89.5 63.5) (end 87.5 65.5) (width 0.3) (layer "F.Cu") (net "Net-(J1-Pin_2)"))
 (segment (start 87.5 65.5) (end 75.5 65.5) (width 0.3) (layer "F.Cu") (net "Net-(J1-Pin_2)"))
 (segment (start 140.5 81) (end 141.5 81) (width 0.3) (layer "F.Cu") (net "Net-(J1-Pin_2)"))
 (segment (start 89.5 60.035) (end 95.1775 60.035) (width 0.3) (layer "F.Cu") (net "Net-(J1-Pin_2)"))
 (segment (start 141.5 81) (end 141.535 80.965) (width 0.3) (layer "F.Cu") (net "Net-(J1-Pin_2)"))
 (segment (start 141.535 80.965) (end 148.6725 80.965) (width 0.3) (layer "F.Cu") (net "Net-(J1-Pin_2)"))
 (segment (start 95.1775 60.035) (end 95.2125 60) (width 0.2) (layer "F.Cu") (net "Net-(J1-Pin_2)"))
 (segment (start 81.8275 60.035) (end 89.5 60.035) (width 0.3) (layer "F.Cu") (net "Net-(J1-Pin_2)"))
 (segment (start 140.5 93.5) (end 140.5 81) (width 0.3) (layer "F.Cu") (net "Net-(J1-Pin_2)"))
 (segment (start 75.5 65.5) (end 75.5 93.5) (width 0.3) (layer "F.Cu") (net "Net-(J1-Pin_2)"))
 (segment (start 89.5 60.035) (end 89.5 63.5) (width 0.3) (layer "F.Cu") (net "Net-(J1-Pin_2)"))
 (segment (start 122.77 85.5) (end 128.495 85.5) (width 0.2) (layer "F.Cu") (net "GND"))
 (segment (start 131.23 76.36) (end 128.495 79.095) (width 0.2) (layer "F.Cu") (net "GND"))
 (segment (start 128.495 85.5) (end 130.995 88) (width 0.2) (layer "F.Cu") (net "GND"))
 (segment (start 116.27 85.5) (end 122.77 85.5) (width 0.2) (layer "F.Cu") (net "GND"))
 (segment (start 128.495 79.095) (end 128.495 85.5) (width 0.2) (layer "F.Cu") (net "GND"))
 (segment (start 110.96 87) (end 127.595 87) (width 0.2) (layer "F.Cu") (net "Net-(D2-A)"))
 (segment (start 129.795 89.2) (end 132.335 89.2) (width 0.2) (layer "F.Cu") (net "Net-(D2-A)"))
 (segment (start 127.595 87) (end 129.795 89.2) (width 0.2) (layer "F.Cu") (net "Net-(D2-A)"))
 (segment (start 98.84 74.88) (end 110.96 87) (width 0.2) (layer "F.Cu") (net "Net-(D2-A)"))
 (segment (start 132.335 89.2) (end 133.535 88) (width 0.2) (layer "F.Cu") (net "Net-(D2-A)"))
 (segment (start 103.6 77.1) (end 101.38 74.88) (width 0.2) (layer "F.Cu") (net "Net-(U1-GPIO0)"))
 (segment (start 124.85 76) (end 123.75 77.1) (width 0.2) (layer "F.Cu") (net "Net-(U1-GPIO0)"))
 (segment (start 123.75 77.1) (end 103.6 77.1) (width 0.2) (layer "F.Cu") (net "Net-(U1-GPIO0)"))
 (segment (start 111.42 90) (end 116.27 90) (width 0.2) (layer "F.Cu") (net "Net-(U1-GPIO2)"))
 (segment (start 116.27 90) (end 122.77 90) (width 0.2) (layer "F.Cu") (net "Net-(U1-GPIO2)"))
 (segment (start 96.3 74.88) (end 111.42 90) (width 0.2) (layer "F.Cu") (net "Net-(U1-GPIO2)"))
 (segment (start 83.6 74.88) (end 93.48 65) (width 0.2) (layer "F.Cu") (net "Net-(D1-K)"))
 (segment (start 146.5 64.5) (end 150 68) (width 0.2) (layer "F.Cu") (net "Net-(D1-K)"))
 (segment (start 146.5 53.5) (end 146.5 64.5) (width 0.2) (layer "F.Cu") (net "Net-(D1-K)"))
 (segment (start 93.48 65) (end 124.2925 65) (width 0.2) (layer "F.Cu") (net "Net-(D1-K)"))
 (segment (start 124.2925 65) (end 139 65) (width 0.2) (layer "F.Cu") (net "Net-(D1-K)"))
 (segment (start 141 65) (end 146 65) (width 0.2) (layer "F.Cu") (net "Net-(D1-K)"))
 (segment (start 137.9 48) (end 141 48) (width 0.2) (layer "F.Cu") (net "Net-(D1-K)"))
 (segment (start 141 48) (end 146.5 53.5) (width 0.2) (layer "F.Cu") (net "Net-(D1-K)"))
 (segment (start 146 65) (end 146.5 64.5) (width 0.2) (layer "F.Cu") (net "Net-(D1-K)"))
 (via (at 139 65) (size 0.6) (drill 0.3) (layers "F.Cu" "B.Cu") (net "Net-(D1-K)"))
 (via (at 141 65) (size 0.6) (drill 0.3) (layers "F.Cu" "B.Cu") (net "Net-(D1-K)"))
 (segment (start 139 65) (end 141 65) (width 0.2) (layer "B.Cu") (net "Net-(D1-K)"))
 (segment (start 86.14 74.88) (end 95.02 66) (width 0.2) (layer "F.Cu") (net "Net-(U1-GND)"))
 (segment (start 111.0925 64.4) (end 124.2925 51.2) (width 0.2) (layer "F.Cu") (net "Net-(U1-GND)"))
 (segment (start 124.2925 51.2) (end 124.2925 50) (width 0.2) (layer "F.Cu") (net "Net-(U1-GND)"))
 (segment (start 107.5 64.4) (end 111.0925 64.4) (width 0.2) (layer "F.Cu") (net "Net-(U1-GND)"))
 (segment (start 95.02 66) (end 106 66) (width 0.2) (layer "F.Cu") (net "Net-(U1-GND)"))
 (via (at 107.5 64.4) (size 0.6) (drill 0.3) (layers "F.Cu" "B.Cu") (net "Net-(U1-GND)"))
 (via (at 106 66) (size 0.6) (drill 0.3) (layers "F.Cu" "B.Cu") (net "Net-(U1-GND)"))
 (segment (start 107.5 64.5) (end 107.5 64.4) (width 0.2) (layer "B.Cu") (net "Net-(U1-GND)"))
 (segment (start 106 66) (end 107.5 64.5) (width 0.2) (layer "B.Cu") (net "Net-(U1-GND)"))
 (segment (start 133.77 74.07) (end 139.84 68) (width 0.2) (layer "F.Cu") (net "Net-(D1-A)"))
 (segment (start 139.84 61.94) (end 137.9 60) (width 0.2) (layer "F.Cu") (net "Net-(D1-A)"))
 (segment (start 139.84 68) (end 139.84 61.94) (width 0.2) (layer "F.Cu") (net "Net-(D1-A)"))
 (segment (start 133.77 76.36) (end 133.77 74.07) (width 0.2) (layer "F.Cu") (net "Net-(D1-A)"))
 (segment (start 130.59 73.5) (end 132.5 75.41) (width 0.2) (layer "F.Cu") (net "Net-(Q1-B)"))
 (segment (start 114.69 76) (end 114.69 73.81) (width 0.2) (layer "F.Cu") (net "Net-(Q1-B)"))
 (segment (start 114.69 73.81) (end 115 73.5) (width 0.2) (layer "F.Cu") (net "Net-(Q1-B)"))
 (segment (start 115 73.5) (end 130.59 73.5) (width 0.2) (layer "F.Cu") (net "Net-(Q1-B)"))
 (segment (start 132.5 75.41) (end 132.5 76.36) (width 0.2) (layer "F.Cu") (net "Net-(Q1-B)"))
 (segment (start 81.8275 54.955) (end 89.5 54.955) (width 0.3) (layer "F.Cu") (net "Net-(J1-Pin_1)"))
 (segment (start 131 44.5) (end 91 44.5) (width 0.3) (layer "F.Cu") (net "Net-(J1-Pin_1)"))
 (segment (start 135.9 54) (end 131 49.1) (width 0.3) (layer "F.Cu") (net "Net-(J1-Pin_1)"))
 (segment (start 89.5 54.955) (end 95.1675 54.955) (width 0.3) (layer "F.Cu") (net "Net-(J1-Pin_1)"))
 (segment (start 91 44.5) (end 89.5 46) (width 0.3) (layer "F.Cu") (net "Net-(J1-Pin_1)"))
 (segment (start 95.1675 54.955) (end 95.2125 55) (width 0.2) (layer "F.Cu") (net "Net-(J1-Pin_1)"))
 (segment (start 89.5 46) (end 89.5 54.955) (width 0.3) (layer "F.Cu") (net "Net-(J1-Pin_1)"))
 (segment (start 131 49.1) (end 131 44.5) (width 0.3) (layer "F.Cu") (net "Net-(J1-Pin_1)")))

